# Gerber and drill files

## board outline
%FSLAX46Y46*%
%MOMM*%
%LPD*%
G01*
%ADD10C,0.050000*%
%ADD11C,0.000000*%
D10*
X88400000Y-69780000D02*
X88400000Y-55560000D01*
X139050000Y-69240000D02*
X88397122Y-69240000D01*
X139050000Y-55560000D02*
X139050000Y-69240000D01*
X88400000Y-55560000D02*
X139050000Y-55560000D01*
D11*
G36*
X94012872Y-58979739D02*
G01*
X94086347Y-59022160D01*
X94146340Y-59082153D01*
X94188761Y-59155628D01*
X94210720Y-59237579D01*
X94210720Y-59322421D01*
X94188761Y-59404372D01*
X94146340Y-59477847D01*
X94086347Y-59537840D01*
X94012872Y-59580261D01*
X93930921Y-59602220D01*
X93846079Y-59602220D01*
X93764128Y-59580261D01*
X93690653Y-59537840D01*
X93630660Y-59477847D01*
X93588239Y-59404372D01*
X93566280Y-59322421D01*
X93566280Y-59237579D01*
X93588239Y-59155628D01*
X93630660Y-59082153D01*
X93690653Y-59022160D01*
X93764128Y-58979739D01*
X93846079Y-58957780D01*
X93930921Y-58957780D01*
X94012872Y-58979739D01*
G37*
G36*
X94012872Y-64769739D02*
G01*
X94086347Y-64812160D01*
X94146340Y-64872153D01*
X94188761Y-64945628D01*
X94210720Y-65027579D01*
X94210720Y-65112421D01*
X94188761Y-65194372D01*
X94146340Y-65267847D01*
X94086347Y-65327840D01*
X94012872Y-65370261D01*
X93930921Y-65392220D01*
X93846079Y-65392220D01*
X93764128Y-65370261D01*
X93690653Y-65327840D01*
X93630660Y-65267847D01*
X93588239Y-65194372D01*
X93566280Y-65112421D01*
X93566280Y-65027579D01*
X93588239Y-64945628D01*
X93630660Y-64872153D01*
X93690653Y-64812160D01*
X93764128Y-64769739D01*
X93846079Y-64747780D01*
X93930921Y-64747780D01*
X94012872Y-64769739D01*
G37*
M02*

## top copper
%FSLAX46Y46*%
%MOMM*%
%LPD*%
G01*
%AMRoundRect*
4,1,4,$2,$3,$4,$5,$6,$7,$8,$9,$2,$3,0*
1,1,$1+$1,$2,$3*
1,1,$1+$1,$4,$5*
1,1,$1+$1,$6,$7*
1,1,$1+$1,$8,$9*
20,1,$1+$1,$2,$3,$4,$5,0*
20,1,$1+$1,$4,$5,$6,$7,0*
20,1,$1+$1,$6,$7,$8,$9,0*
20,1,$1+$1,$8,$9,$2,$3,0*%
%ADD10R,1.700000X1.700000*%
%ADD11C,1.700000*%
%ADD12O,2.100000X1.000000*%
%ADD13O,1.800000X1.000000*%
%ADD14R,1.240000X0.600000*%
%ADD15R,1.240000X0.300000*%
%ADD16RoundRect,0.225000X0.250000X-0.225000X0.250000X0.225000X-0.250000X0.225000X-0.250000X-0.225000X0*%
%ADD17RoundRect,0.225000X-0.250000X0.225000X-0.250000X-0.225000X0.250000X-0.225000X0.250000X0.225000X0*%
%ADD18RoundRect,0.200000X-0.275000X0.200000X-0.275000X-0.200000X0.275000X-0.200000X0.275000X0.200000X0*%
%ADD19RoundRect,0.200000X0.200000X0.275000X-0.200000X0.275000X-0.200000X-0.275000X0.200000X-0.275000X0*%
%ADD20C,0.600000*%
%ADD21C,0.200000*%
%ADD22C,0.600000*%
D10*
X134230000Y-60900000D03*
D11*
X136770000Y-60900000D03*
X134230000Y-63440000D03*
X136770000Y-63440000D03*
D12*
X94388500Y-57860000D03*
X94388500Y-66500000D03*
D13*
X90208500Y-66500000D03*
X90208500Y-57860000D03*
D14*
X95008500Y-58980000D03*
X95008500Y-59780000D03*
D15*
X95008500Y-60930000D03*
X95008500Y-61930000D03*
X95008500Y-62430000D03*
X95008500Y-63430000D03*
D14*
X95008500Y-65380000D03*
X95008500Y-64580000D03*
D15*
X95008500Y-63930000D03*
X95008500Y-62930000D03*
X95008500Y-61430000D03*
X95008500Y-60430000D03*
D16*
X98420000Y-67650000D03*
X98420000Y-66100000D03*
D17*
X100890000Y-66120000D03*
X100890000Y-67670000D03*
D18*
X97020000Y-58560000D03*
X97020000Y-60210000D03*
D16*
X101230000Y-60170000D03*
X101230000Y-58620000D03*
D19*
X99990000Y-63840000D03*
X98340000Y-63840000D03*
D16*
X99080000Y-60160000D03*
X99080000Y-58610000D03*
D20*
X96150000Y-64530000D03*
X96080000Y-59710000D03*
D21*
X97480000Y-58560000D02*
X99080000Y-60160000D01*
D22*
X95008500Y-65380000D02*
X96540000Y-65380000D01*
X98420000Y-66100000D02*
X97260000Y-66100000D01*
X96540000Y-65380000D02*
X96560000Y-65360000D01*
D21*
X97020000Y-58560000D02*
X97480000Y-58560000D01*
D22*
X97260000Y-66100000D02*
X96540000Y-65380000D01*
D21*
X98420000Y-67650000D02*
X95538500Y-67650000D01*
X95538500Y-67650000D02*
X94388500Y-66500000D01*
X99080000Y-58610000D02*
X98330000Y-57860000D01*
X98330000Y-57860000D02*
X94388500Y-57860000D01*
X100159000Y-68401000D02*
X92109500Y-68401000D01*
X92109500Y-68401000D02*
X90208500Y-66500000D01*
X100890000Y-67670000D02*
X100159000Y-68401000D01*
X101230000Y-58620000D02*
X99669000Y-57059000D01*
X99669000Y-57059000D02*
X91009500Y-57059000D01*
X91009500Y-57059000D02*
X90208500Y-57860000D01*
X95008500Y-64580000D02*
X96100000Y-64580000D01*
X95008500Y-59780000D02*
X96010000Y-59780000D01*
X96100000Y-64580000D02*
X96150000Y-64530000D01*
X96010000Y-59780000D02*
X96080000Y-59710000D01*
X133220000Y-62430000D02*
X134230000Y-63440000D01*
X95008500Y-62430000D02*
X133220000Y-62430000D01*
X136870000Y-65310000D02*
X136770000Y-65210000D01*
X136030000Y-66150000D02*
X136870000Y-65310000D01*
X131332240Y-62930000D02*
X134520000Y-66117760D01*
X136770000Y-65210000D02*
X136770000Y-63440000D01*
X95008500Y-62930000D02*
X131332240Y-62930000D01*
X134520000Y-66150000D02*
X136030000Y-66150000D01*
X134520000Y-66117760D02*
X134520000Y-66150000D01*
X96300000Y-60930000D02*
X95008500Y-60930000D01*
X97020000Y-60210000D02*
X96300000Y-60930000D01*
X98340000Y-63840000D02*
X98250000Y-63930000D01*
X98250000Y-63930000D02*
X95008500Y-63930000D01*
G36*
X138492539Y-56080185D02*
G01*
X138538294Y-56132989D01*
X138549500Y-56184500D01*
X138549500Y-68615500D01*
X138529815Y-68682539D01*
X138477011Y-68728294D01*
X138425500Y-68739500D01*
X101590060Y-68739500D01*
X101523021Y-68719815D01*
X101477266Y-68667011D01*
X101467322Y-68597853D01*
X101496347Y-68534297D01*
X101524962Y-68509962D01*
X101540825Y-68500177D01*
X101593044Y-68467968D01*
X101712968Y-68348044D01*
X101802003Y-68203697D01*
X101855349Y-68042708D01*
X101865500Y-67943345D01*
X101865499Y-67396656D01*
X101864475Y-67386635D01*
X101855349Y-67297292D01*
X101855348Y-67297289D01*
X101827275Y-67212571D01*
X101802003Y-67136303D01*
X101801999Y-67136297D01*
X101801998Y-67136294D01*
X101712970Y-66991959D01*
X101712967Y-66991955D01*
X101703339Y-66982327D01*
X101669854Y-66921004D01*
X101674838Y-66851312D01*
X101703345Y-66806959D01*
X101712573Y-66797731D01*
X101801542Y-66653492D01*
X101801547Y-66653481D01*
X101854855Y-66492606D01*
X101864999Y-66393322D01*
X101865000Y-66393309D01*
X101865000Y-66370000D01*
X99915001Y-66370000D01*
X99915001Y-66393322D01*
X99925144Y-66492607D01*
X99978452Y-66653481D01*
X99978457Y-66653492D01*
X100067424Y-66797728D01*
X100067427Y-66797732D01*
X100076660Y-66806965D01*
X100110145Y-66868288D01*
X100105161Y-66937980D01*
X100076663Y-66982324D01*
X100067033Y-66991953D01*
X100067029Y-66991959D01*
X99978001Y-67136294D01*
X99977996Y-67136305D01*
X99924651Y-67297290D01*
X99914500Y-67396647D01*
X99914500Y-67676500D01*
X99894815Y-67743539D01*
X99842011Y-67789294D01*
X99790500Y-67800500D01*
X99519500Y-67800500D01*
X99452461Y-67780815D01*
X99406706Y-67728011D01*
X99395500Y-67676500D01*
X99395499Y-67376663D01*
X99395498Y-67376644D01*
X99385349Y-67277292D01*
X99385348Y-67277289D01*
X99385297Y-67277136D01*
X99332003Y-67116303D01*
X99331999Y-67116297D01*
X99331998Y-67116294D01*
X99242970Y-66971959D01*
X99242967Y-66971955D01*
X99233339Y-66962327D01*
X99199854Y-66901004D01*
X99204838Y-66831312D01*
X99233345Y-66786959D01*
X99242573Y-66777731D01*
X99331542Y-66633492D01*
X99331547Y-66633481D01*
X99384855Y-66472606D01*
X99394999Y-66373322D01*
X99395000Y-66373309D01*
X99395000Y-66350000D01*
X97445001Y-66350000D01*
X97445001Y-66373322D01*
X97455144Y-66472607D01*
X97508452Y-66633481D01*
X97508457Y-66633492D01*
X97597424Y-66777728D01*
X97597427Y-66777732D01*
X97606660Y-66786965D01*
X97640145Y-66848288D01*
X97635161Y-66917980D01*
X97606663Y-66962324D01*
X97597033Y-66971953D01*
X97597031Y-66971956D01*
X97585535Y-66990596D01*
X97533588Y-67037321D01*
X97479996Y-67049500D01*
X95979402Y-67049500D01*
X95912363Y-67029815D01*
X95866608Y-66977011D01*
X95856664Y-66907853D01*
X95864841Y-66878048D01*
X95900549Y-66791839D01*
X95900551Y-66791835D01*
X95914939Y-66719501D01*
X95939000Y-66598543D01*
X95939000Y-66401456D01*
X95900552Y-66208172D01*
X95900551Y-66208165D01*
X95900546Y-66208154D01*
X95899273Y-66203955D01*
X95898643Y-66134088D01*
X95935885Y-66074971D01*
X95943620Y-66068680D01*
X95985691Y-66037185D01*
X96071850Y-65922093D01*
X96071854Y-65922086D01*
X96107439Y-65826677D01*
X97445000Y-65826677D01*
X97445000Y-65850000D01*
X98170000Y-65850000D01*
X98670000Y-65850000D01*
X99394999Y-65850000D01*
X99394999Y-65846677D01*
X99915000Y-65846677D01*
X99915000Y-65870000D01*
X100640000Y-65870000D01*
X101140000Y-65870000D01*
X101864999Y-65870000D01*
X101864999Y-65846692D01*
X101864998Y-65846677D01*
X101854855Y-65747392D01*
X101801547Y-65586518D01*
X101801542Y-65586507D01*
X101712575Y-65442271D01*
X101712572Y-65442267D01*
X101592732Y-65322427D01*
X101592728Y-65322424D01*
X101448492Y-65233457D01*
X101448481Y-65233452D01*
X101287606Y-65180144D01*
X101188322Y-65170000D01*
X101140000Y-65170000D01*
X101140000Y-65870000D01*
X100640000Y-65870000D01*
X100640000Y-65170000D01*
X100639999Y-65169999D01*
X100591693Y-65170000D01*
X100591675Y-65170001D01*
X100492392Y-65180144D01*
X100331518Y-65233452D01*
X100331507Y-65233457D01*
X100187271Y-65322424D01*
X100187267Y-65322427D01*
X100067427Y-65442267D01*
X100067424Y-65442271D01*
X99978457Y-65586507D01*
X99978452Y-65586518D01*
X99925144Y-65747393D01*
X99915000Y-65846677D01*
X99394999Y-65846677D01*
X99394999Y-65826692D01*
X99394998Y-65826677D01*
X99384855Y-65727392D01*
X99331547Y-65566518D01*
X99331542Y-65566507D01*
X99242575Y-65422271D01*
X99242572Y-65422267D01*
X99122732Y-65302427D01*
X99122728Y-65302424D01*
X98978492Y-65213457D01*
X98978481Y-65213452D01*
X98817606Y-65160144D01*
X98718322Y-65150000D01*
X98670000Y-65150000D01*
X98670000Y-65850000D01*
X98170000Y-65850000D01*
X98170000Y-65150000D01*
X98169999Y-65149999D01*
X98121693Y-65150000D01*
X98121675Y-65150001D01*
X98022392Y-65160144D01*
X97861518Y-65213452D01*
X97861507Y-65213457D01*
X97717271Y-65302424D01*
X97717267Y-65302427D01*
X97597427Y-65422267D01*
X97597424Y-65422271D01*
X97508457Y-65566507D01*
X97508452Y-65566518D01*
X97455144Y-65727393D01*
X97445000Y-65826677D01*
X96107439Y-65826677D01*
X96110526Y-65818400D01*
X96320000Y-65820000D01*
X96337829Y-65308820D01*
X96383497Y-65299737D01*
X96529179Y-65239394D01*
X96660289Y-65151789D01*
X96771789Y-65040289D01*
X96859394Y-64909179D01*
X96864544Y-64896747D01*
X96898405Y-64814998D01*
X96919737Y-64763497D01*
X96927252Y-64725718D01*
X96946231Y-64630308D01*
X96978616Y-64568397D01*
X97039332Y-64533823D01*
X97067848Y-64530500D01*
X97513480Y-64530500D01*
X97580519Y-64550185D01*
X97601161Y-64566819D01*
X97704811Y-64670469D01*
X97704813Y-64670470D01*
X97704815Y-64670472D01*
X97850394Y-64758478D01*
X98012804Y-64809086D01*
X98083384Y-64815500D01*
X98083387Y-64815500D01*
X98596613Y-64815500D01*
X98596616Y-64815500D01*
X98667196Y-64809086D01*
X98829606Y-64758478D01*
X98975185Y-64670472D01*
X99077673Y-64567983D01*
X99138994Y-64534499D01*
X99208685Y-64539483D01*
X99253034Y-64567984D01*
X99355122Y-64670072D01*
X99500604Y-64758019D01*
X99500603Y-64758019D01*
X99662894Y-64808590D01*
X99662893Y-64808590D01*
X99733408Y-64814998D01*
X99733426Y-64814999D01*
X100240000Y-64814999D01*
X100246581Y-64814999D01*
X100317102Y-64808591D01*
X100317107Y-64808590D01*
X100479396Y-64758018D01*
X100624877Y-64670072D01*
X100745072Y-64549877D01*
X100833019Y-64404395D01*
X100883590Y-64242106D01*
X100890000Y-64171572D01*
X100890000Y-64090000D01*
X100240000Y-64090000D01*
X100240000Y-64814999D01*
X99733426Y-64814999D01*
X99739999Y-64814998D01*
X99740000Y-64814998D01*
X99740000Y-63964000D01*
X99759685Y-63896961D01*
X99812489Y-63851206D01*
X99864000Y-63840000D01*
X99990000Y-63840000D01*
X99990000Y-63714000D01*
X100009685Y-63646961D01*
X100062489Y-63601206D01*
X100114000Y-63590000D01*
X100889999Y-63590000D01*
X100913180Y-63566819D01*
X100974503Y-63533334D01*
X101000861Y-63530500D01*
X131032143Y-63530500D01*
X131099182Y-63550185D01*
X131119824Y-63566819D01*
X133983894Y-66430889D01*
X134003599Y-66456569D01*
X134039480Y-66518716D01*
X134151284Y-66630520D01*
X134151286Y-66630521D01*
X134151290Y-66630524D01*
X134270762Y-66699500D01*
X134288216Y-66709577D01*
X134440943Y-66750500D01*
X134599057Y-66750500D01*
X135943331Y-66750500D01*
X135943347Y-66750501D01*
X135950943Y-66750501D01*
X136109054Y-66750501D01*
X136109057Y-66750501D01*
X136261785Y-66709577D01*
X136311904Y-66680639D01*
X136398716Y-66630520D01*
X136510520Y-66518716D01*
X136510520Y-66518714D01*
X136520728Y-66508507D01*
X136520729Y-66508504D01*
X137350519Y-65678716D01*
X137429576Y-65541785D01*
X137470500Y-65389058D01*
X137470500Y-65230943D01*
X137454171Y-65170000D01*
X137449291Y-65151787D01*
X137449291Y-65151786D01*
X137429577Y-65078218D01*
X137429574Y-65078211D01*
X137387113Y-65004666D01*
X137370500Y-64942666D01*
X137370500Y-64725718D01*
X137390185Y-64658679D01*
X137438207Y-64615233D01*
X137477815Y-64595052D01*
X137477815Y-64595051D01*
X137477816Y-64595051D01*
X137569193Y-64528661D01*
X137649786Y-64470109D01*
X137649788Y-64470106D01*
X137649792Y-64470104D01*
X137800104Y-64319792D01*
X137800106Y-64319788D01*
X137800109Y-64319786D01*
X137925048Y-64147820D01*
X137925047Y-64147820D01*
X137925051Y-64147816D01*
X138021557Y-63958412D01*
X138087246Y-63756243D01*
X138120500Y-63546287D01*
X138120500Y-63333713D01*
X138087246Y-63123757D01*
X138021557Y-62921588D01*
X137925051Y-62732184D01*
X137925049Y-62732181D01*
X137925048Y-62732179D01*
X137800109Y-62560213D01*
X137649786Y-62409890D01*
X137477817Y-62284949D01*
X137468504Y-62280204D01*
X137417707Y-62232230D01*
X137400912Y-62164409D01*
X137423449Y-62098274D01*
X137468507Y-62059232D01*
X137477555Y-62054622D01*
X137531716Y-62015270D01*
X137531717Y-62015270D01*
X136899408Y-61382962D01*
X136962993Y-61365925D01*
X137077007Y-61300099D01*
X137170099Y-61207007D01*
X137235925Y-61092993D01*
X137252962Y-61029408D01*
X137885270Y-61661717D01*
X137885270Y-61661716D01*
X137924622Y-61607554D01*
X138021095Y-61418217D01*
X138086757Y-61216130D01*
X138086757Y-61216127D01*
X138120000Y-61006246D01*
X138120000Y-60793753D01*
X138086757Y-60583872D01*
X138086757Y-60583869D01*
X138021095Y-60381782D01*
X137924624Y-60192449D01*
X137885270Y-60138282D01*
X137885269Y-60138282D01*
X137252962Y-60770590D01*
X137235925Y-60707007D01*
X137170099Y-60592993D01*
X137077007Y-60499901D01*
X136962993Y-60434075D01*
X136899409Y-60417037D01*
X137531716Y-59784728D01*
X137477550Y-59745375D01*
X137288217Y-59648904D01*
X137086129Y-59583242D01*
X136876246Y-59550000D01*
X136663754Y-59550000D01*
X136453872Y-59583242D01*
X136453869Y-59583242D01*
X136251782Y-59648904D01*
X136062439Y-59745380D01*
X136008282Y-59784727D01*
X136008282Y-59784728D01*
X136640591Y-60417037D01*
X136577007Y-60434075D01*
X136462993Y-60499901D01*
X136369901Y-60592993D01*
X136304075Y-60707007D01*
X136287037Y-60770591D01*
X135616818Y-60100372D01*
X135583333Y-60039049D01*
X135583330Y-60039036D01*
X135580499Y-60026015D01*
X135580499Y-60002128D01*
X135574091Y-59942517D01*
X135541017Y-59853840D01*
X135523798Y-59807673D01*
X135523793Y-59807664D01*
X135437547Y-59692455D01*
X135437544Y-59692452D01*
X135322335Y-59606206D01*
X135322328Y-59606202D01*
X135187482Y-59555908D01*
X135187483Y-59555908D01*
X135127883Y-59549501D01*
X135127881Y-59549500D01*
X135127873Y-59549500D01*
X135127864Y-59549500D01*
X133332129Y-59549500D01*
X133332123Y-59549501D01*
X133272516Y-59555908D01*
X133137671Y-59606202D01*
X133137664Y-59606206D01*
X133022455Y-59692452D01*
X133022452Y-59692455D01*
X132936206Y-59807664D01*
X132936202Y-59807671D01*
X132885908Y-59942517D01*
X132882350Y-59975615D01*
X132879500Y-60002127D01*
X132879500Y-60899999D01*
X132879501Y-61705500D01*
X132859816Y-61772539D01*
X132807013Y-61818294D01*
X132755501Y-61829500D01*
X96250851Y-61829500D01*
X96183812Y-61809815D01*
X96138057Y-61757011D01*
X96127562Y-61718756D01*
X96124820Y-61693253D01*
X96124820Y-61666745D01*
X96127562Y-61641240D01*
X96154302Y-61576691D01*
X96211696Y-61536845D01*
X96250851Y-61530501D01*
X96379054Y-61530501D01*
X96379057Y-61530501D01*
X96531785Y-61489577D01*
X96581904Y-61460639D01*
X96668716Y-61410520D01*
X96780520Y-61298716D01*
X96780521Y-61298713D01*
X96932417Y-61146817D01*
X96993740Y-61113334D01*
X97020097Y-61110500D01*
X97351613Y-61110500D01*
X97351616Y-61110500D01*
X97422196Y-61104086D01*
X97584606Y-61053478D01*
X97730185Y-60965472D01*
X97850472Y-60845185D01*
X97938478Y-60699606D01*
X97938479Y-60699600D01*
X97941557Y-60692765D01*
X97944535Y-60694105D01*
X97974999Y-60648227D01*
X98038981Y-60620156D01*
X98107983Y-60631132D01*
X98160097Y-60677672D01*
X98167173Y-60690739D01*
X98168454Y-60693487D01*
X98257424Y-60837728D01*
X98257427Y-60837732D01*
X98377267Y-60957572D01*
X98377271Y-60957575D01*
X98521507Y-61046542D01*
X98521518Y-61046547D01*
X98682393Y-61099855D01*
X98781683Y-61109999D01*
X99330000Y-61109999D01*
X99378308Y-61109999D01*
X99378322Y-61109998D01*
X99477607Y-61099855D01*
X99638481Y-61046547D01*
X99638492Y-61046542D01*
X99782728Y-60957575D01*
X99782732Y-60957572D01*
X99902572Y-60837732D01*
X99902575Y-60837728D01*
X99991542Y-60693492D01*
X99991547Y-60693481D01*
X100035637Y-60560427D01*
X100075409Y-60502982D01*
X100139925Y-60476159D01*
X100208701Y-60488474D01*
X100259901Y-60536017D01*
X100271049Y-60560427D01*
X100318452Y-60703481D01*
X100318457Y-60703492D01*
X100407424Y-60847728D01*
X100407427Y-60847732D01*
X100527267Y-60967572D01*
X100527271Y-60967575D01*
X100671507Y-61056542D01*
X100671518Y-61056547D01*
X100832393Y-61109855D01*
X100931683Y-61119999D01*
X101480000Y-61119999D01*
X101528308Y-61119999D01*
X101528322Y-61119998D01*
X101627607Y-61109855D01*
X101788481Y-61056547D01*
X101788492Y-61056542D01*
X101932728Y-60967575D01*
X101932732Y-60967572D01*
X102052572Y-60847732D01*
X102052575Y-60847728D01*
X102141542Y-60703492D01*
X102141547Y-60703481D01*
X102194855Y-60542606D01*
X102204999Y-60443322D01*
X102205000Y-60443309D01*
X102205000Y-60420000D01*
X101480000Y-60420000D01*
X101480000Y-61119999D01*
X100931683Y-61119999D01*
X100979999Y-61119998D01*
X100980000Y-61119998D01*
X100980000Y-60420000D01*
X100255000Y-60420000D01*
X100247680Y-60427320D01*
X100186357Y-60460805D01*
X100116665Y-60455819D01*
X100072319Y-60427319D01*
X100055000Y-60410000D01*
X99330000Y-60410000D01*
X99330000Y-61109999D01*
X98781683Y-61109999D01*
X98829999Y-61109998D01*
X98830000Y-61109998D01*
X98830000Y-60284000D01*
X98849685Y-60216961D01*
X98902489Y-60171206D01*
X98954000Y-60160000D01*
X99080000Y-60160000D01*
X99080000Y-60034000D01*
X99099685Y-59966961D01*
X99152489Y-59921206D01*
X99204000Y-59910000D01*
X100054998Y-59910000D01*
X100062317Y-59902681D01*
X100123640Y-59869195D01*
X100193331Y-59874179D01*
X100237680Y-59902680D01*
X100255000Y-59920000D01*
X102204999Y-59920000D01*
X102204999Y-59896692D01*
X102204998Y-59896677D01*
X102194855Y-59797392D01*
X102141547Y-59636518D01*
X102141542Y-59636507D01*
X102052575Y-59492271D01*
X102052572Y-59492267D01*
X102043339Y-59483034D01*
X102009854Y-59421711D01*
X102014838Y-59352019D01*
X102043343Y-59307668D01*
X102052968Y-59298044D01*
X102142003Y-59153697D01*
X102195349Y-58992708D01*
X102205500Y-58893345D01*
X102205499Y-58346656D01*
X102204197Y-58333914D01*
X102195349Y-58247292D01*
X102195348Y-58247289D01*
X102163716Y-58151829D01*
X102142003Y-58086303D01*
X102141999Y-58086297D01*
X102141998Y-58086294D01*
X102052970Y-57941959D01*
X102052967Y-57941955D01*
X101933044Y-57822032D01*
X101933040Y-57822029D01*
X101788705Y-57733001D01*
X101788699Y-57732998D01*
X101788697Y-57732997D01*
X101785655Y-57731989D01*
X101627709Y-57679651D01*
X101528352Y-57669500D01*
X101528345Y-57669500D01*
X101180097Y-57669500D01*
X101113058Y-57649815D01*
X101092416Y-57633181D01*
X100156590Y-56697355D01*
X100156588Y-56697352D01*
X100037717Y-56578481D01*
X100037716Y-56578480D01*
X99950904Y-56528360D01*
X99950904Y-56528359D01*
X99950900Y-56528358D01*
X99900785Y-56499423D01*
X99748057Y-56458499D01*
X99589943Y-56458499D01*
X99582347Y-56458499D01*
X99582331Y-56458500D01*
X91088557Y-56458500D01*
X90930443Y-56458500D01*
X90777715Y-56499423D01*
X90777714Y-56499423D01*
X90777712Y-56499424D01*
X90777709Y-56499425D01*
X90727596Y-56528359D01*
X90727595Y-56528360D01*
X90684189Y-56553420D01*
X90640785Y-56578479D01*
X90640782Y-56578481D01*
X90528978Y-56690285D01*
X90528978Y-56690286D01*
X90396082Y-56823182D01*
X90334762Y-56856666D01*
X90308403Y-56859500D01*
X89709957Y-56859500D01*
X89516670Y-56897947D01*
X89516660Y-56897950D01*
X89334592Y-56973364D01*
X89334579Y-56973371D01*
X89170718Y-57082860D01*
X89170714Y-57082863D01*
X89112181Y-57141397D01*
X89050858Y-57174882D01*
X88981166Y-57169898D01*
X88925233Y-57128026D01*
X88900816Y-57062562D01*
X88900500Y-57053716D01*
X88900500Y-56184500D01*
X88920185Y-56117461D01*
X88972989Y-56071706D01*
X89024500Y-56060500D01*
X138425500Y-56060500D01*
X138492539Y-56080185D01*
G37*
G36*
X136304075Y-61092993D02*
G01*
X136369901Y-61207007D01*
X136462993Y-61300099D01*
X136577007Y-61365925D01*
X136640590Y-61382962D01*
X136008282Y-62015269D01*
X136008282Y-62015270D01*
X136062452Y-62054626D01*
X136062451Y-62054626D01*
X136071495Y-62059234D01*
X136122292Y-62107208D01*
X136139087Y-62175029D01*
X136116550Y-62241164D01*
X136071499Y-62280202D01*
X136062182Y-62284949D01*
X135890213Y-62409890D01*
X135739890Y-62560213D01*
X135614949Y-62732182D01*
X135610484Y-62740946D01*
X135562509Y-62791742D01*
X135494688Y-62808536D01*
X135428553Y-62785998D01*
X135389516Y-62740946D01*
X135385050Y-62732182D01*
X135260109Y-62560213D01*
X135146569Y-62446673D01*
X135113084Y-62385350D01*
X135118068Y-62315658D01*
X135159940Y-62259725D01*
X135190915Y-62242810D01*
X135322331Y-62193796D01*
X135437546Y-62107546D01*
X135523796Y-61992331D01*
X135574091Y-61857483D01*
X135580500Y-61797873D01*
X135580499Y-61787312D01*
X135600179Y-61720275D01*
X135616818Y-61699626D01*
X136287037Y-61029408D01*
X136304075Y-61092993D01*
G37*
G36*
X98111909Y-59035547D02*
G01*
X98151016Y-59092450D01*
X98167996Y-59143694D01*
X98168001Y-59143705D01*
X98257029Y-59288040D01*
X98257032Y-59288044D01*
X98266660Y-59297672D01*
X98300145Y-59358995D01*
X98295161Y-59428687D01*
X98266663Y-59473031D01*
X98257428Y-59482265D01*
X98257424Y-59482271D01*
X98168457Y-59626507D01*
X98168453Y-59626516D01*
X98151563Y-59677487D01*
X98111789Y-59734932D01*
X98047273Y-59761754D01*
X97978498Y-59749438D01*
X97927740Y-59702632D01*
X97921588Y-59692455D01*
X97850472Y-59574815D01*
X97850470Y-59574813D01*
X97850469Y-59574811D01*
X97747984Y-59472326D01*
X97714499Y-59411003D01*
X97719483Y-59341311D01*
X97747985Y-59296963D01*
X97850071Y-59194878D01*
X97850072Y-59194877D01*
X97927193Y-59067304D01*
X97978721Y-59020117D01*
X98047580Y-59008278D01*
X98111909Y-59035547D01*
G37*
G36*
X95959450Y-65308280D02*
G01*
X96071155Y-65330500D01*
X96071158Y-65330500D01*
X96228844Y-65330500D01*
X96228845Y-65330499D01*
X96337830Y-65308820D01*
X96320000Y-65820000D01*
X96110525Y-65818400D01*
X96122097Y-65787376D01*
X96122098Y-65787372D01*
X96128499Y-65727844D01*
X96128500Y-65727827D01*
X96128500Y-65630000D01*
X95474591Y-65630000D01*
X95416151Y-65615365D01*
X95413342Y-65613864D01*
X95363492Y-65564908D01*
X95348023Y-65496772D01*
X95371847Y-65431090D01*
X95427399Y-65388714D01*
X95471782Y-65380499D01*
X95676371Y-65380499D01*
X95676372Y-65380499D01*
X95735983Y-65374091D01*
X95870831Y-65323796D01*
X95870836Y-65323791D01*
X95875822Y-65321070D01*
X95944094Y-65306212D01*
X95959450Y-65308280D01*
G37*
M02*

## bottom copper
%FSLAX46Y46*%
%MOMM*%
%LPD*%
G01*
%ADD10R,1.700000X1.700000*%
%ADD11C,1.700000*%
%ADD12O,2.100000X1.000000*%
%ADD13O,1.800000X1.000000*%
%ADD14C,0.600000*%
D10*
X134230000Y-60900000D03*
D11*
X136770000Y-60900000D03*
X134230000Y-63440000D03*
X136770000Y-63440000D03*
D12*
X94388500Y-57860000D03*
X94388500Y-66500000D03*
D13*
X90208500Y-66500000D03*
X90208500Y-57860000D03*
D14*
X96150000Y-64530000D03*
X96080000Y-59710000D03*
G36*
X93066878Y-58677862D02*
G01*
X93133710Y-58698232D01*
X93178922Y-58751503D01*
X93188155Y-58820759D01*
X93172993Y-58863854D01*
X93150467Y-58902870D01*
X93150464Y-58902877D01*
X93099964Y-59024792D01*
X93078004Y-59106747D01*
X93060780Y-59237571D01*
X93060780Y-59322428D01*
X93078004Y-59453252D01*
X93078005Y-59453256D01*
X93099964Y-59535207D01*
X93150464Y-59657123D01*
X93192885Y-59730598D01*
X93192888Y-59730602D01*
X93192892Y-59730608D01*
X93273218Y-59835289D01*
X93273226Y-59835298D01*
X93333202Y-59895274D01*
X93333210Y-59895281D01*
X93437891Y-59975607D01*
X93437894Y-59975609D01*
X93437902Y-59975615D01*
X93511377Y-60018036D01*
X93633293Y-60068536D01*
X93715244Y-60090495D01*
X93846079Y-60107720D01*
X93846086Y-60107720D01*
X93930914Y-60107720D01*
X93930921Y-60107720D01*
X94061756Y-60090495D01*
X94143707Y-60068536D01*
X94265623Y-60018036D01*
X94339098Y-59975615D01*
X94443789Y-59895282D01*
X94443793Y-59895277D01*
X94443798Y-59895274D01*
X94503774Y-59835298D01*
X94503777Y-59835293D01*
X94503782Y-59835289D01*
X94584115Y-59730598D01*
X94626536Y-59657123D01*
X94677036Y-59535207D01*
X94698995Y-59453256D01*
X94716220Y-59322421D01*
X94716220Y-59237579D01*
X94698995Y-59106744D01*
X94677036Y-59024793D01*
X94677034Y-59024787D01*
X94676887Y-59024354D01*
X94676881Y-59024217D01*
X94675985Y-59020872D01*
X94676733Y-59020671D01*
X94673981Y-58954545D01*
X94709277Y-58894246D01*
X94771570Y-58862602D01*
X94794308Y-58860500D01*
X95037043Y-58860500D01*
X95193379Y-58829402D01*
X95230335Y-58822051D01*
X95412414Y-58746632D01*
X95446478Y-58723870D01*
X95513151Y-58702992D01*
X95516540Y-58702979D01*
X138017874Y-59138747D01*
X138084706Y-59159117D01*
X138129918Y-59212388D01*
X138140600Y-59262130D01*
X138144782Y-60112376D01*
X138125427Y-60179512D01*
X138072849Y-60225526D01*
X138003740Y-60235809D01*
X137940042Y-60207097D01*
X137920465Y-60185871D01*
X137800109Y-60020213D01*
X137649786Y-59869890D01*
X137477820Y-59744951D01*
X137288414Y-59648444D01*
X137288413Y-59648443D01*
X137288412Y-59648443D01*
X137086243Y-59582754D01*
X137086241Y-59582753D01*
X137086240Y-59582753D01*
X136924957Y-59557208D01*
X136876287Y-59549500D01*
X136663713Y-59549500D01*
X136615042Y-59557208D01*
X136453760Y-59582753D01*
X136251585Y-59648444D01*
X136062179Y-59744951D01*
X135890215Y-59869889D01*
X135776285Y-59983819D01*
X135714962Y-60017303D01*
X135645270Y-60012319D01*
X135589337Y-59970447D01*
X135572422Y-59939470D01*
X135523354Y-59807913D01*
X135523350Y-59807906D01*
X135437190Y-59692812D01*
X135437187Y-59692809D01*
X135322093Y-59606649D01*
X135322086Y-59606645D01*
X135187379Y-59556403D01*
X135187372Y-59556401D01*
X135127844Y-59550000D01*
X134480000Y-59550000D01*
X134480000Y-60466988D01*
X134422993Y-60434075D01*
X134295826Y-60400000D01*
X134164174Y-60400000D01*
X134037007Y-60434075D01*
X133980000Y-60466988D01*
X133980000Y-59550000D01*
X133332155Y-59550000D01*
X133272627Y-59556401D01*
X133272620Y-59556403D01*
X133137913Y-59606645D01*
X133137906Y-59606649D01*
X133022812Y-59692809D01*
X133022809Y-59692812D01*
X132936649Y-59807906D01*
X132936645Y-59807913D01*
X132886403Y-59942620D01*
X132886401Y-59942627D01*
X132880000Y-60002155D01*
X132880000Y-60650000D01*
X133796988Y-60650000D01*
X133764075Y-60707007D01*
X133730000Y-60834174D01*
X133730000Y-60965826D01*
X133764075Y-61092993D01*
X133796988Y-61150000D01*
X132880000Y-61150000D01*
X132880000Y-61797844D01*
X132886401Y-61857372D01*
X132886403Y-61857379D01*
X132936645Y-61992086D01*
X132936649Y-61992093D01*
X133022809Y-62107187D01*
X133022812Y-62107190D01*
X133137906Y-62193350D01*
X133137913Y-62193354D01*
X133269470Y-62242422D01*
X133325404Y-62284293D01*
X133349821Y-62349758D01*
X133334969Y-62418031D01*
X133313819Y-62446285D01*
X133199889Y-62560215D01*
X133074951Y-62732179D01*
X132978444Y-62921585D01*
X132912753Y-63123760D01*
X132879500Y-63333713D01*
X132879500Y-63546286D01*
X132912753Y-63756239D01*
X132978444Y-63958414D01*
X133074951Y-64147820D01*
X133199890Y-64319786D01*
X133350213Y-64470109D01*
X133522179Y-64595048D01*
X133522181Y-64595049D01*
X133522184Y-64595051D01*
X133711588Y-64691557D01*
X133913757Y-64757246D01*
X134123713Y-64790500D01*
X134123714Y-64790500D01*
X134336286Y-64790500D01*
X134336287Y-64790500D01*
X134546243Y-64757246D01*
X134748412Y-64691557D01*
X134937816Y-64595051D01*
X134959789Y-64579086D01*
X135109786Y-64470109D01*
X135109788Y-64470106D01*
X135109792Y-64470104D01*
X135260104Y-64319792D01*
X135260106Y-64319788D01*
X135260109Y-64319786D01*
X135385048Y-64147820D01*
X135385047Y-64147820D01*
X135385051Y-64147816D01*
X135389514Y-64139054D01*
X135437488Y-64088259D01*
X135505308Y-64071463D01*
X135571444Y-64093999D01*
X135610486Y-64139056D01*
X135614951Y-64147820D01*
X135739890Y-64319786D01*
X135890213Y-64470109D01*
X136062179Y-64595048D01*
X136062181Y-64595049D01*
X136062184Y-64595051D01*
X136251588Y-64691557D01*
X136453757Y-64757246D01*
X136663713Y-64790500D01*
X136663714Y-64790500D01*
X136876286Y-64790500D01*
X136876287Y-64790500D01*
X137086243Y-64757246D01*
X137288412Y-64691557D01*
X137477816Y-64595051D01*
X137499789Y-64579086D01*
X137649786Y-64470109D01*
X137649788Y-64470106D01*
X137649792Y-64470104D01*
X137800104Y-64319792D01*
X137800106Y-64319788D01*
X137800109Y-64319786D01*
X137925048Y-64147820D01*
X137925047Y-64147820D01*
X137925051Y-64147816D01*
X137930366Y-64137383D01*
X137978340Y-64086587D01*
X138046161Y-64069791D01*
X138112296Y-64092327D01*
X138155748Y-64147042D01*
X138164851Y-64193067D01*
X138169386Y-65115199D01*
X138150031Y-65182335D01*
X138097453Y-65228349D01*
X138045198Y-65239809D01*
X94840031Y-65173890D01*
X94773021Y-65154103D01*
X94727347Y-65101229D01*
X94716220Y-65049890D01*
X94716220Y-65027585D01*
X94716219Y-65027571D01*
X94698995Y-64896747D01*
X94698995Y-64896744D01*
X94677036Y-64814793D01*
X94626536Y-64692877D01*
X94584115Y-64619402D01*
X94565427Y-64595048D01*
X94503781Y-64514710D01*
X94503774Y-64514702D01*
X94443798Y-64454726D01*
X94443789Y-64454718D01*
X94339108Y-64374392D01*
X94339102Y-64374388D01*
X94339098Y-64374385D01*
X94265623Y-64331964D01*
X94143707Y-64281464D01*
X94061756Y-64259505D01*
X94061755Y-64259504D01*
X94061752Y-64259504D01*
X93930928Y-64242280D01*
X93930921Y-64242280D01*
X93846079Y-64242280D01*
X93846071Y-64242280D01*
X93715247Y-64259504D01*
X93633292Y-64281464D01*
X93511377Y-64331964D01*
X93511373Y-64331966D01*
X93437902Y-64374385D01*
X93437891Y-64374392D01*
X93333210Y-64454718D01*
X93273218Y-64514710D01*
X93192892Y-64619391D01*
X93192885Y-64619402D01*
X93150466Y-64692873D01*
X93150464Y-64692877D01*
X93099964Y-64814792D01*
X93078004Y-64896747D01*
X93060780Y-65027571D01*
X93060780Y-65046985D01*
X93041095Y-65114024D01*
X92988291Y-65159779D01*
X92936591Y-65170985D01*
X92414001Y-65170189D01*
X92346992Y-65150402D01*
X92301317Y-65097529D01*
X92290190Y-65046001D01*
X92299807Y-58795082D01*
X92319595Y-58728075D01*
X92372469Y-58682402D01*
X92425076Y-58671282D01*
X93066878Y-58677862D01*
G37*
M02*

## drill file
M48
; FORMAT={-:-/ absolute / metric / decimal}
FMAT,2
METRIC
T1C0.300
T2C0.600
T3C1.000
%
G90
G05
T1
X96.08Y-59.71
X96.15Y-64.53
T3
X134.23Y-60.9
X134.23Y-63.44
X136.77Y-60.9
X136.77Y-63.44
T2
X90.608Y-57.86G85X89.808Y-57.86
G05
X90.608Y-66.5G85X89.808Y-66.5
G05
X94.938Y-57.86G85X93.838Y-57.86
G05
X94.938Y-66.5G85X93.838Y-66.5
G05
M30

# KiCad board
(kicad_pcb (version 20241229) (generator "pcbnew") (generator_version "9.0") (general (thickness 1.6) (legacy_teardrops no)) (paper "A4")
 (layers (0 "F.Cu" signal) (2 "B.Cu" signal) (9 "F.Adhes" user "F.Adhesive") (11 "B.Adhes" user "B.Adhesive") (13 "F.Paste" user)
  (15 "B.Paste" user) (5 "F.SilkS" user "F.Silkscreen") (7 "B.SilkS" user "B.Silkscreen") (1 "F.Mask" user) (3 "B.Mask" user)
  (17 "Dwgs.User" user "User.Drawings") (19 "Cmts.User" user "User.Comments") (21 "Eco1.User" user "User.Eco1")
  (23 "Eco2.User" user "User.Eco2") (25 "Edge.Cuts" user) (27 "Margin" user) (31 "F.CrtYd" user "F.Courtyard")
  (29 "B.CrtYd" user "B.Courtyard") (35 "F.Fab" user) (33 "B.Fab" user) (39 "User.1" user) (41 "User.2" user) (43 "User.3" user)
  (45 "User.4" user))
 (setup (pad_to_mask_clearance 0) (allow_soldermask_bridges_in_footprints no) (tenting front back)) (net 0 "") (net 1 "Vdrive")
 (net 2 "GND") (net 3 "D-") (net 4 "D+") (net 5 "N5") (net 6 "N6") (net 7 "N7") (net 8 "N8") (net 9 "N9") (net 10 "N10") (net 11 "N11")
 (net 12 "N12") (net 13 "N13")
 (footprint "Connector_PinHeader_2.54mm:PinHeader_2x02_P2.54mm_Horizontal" (layer "F.Cu") (at 134.23 60.9)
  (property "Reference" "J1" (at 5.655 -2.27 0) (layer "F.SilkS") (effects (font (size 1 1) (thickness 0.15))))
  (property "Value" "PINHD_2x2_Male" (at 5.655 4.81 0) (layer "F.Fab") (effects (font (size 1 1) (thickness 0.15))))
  (pad "1" thru_hole rect (at 0 0) (size 1.7 1.7) (drill 1) (layers "*.Cu" "*.Mask") (remove_unused_layers no) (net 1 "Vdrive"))
  (pad "2" thru_hole circle (at 2.54 0) (size 1.7 1.7) (drill 1) (layers "*.Cu" "*.Mask") (remove_unused_layers no) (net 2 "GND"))
  (pad "3" thru_hole circle (at 0 2.54) (size 1.7 1.7) (drill 1) (layers "*.Cu" "*.Mask") (remove_unused_layers no) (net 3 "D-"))
  (pad "4" thru_hole circle (at 2.54 2.54) (size 1.7 1.7) (drill 1) (layers "*.Cu" "*.Mask") (remove_unused_layers no) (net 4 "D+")))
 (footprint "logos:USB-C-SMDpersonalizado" (layer "F.Cu") (at 92.6085 62.18 -90)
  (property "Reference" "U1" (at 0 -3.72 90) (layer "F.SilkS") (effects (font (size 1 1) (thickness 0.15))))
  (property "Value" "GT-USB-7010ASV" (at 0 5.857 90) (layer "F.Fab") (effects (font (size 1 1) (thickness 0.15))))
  (fp_poly
   (pts (xy -2.57778 -1.322421) (xy -2.599739 -1.404372) (xy -2.64216 -1.477847) (xy -2.702153 -1.53784) (xy -2.775628 -1.580261)
    (xy -2.857579 -1.60222) (xy -2.942421 -1.60222) (xy -3.024372 -1.580261) (xy -3.097847 -1.53784) (xy -3.15784 -1.477847)
    (xy -3.200261 -1.404372) (xy -3.22222 -1.322421) (xy -3.22222 -1.237579) (xy -3.200261 -1.155628) (xy -3.15784 -1.082153)
    (xy -3.097847 -1.02216) (xy -3.024372 -0.979739) (xy -2.942421 -0.95778) (xy -2.857579 -0.95778) (xy -2.775628 -0.979739)
    (xy -2.702153 -1.02216) (xy -2.64216 -1.082153) (xy -2.599739 -1.155628) (xy -2.57778 -1.237579))
   (stroke (width 0) (type default)) (fill yes) (layer "Edge.Cuts"))
  (fp_poly
   (pts (xy 3.21222 -1.322421) (xy 3.190261 -1.404372) (xy 3.14784 -1.477847) (xy 3.087847 -1.53784) (xy 3.014372 -1.580261)
    (xy 2.932421 -1.60222) (xy 2.847579 -1.60222) (xy 2.765628 -1.580261) (xy 2.692153 -1.53784) (xy 2.63216 -1.477847)
    (xy 2.589739 -1.404372) (xy 2.56778 -1.322421) (xy 2.56778 -1.237579) (xy 2.589739 -1.155628) (xy 2.63216 -1.082153)
    (xy 2.692153 -1.02216) (xy 2.765628 -0.979739) (xy 2.847579 -0.95778) (xy 2.932421 -0.95778) (xy 3.014372 -0.979739)
    (xy 3.087847 -1.02216) (xy 3.14784 -1.082153) (xy 3.190261 -1.155628) (xy 3.21222 -1.237579))
   (stroke (width 0) (type default)) (fill yes) (layer "Edge.Cuts"))
  (pad "1" thru_hole oval (at -4.32 -1.78 270) (size 1 2.1) (drill oval 0.6 1.7) (layers "*.Cu" "*.Mask") (remove_unused_layers no)
   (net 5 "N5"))
  (pad "2" thru_hole oval (at 4.32 -1.78 270) (size 1 2.1) (drill oval 0.6 1.7) (layers "*.Cu" "*.Mask") (remove_unused_layers no)
   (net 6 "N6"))
  (pad "3" thru_hole oval (at 4.32 2.4 270) (size 1 1.8) (drill oval 0.6 1.4) (layers "*.Cu" "*.Mask") (remove_unused_layers no)
   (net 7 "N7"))
  (pad "4" thru_hole oval (at -4.32 2.4 270) (size 1 1.8) (drill oval 0.6 1.4) (layers "*.Cu" "*.Mask") (remove_unused_layers no)
   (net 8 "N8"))
  (pad "A1B12" smd rect (at -3.2 -2.4 270) (size 0.6 1.24) (layers "F.Cu" "F.Mask" "F.Paste") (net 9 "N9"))
  (pad "A4B9" smd rect (at -2.4 -2.4 270) (size 0.6 1.24) (layers "F.Cu" "F.Mask" "F.Paste") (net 1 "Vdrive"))
  (pad "A5" smd rect (at -1.25 -2.4 270) (size 0.3 1.24) (layers "F.Cu" "F.Mask" "F.Paste") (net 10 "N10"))
  (pad "A6" smd rect (at -0.25 -2.4 270) (size 0.3 1.24) (layers "F.Cu" "F.Mask" "F.Paste") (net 4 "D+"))
  (pad "A7" smd rect (at 0.25 -2.4 270) (size 0.3 1.24) (layers "F.Cu" "F.Mask" "F.Paste") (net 3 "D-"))
  (pad "A8" smd rect (at 1.25 -2.4 270) (size 0.3 1.24) (layers "F.Cu" "F.Mask" "F.Paste") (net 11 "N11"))
  (pad "B1A12" smd rect (at 3.2 -2.4 270) (size 0.6 1.24) (layers "F.Cu" "F.Mask" "F.Paste") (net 2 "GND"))
  (pad "B4A9" smd rect (at 2.4 -2.4 270) (size 0.6 1.24) (layers "F.Cu" "F.Mask" "F.Paste") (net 1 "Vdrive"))
  (pad "B5" smd rect (at 1.75 -2.4 270) (size 0.3 1.24) (layers "F.Cu" "F.Mask" "F.Paste") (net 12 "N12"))
  (pad "B6" smd rect (at 0.75 -2.4 270) (size 0.3 1.24) (layers "F.Cu" "F.Mask" "F.Paste") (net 4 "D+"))
  (pad "B7" smd rect (at -0.75 -2.4 270) (size 0.3 1.24) (layers "F.Cu" "F.Mask" "F.Paste") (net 3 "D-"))
  (pad "B8" smd rect (at -1.75 -2.4 270) (size 0.3 1.24) (layers "F.Cu" "F.Mask" "F.Paste") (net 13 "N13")))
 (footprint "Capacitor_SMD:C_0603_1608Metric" (layer "F.Cu") (at 98.42 66.875 90)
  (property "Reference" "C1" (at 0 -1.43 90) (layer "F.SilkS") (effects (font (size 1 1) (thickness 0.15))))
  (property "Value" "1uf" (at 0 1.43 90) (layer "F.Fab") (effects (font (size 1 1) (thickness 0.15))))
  (pad "1" smd roundrect (at -0.775 0 90) (size 0.9 0.95) (layers "F.Cu" "F.Mask" "F.Paste") (roundrect_rratio 0.25) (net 6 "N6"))
  (pad "2" smd roundrect (at 0.775 0 90) (size 0.9 0.95) (layers "F.Cu" "F.Mask" "F.Paste") (roundrect_rratio 0.25) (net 2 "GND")))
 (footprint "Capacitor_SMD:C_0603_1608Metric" (layer "F.Cu") (at 100.89 66.895 -90)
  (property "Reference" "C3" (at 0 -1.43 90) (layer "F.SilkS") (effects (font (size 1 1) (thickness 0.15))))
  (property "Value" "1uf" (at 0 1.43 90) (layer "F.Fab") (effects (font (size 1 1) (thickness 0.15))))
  (pad "1" smd roundrect (at -0.775 0 270) (size 0.9 0.95) (layers "F.Cu" "F.Mask" "F.Paste") (roundrect_rratio 0.25) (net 2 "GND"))
  (pad "2" smd roundrect (at 0.775 0 270) (size 0.9 0.95) (layers "F.Cu" "F.Mask" "F.Paste") (roundrect_rratio 0.25) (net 7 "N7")))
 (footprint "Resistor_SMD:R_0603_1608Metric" (layer "F.Cu") (at 97.02 59.385 -90)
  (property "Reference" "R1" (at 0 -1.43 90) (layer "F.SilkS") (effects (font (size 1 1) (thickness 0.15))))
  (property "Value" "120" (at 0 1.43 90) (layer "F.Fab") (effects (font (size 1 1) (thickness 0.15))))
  (pad "1" smd roundrect (at -0.825 0 270) (size 0.8 0.95) (layers "F.Cu" "F.Mask" "F.Paste") (roundrect_rratio 0.25) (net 2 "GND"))
  (pad "2" smd roundrect (at 0.825 0 270) (size 0.8 0.95) (layers "F.Cu" "F.Mask" "F.Paste") (roundrect_rratio 0.25) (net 10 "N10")))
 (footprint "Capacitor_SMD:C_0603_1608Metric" (layer "F.Cu") (at 101.23 59.395 90)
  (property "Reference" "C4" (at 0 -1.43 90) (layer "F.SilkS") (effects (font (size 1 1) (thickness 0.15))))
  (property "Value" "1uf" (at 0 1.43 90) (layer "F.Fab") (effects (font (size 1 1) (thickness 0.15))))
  (pad "1" smd roundrect (at -0.775 0 90) (size 0.9 0.95) (layers "F.Cu" "F.Mask" "F.Paste") (roundrect_rratio 0.25) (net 2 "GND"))
  (pad "2" smd roundrect (at 0.775 0 90) (size 0.9 0.95) (layers "F.Cu" "F.Mask" "F.Paste") (roundrect_rratio 0.25) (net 8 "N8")))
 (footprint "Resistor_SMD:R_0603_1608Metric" (layer "F.Cu") (at 99.165 63.84 180)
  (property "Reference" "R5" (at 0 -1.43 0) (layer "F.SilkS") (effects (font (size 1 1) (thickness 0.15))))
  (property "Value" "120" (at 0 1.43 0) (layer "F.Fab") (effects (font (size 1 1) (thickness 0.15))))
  (pad "1" smd roundrect (at -0.825 0 180) (size 0.8 0.95) (layers "F.Cu" "F.Mask" "F.Paste") (roundrect_rratio 0.25) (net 2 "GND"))
  (pad "2" smd roundrect (at 0.825 0 180) (size 0.8 0.95) (layers "F.Cu" "F.Mask" "F.Paste") (roundrect_rratio 0.25) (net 12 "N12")))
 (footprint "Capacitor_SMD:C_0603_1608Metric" (layer "F.Cu") (at 99.08 59.385 90)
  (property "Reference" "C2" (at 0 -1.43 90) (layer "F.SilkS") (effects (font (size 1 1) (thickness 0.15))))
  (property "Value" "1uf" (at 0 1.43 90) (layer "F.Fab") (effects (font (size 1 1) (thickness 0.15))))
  (pad "1" smd roundrect (at -0.775 0 90) (size 0.9 0.95) (layers "F.Cu" "F.Mask" "F.Paste") (roundrect_rratio 0.25) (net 2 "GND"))
  (pad "2" smd roundrect (at 0.775 0 90) (size 0.9 0.95) (layers "F.Cu" "F.Mask" "F.Paste") (roundrect_rratio 0.25) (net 5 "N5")))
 (gr_line (start 88.4 69.78) (end 88.4 55.56) (stroke (width 0.05) (type default)) (layer "Edge.Cuts"))
 (gr_line (start 139.05 69.24) (end 88.397122 69.24) (stroke (width 0.05) (type solid)) (layer "Edge.Cuts"))
 (gr_line (start 139.05 55.56) (end 139.05 69.24) (stroke (width 0.05) (type default)) (layer "Edge.Cuts"))
 (gr_line (start 88.4 55.56) (end 139.05 55.56) (stroke (width 0.05) (type default)) (layer "Edge.Cuts"))
 (segment (start 97.48 58.56) (end 99.08 60.16) (width 0.2) (layer "F.Cu") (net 2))
 (segment (start 95.0085 65.38) (end 96.54 65.38) (width 0.6) (layer "F.Cu") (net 2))
 (segment (start 98.42 66.1) (end 97.26 66.1) (width 0.6) (layer "F.Cu") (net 2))
 (segment (start 96.54 65.38) (end 96.56 65.36) (width 0.6) (layer "F.Cu") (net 2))
 (segment (start 97.02 58.56) (end 97.48 58.56) (width 0.2) (layer "F.Cu") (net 2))
 (segment (start 97.26 66.1) (end 96.54 65.38) (width 0.6) (layer "F.Cu") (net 2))
 (segment (start 98.42 67.65) (end 95.5385 67.65) (width 0.2) (layer "F.Cu") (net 6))
 (segment (start 95.5385 67.65) (end 94.3885 66.5) (width 0.2) (layer "F.Cu") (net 6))
 (segment (start 99.08 58.61) (end 98.33 57.86) (width 0.2) (layer "F.Cu") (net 5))
 (segment (start 98.33 57.86) (end 94.3885 57.86) (width 0.2) (layer "F.Cu") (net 5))
 (segment (start 100.159 68.401) (end 92.1095 68.401) (width 0.2) (layer "F.Cu") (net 7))
 (segment (start 92.1095 68.401) (end 90.2085 66.5) (width 0.2) (layer "F.Cu") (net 7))
 (segment (start 100.89 67.67) (end 100.159 68.401) (width 0.2) (layer "F.Cu") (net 7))
 (segment (start 101.23 58.62) (end 99.669 57.059) (width 0.2) (layer "F.Cu") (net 8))
 (segment (start 99.669 57.059) (end 91.0095 57.059) (width 0.2) (layer "F.Cu") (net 8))
 (segment (start 91.0095 57.059) (end 90.2085 57.86) (width 0.2) (layer "F.Cu") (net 8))
 (segment (start 95.0085 64.58) (end 96.1 64.58) (width 0.2) (layer "F.Cu") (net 1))
 (segment (start 95.0085 59.78) (end 96.01 59.78) (width 0.2) (layer "F.Cu") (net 1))
 (segment (start 96.1 64.58) (end 96.15 64.53) (width 0.2) (layer "F.Cu") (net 1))
 (segment (start 96.01 59.78) (end 96.08 59.71) (width 0.2) (layer "F.Cu") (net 1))
 (via (at 96.15 64.53) (size 0.6) (drill 0.3) (layers "F.Cu" "B.Cu") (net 1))
 (via (at 96.08 59.71) (size 0.6) (drill 0.3) (layers "F.Cu" "B.Cu") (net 1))
 (segment (start 133.22 62.43) (end 134.23 63.44) (width 0.2) (layer "F.Cu") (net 3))
 (segment (start 95.0085 62.43) (end 133.22 62.43) (width 0.2) (layer "F.Cu") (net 3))
 (segment (start 136.87 65.31) (end 136.77 65.21) (width 0.2) (layer "F.Cu") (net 4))
 (segment (start 136.03 66.15) (end 136.87 65.31) (width 0.2) (layer "F.Cu") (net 4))
 (segment (start 131.33224 62.93) (end 134.52 66.11776) (width 0.2) (layer "F.Cu") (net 4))
 (segment (start 136.77 65.21) (end 136.77 63.44) (width 0.2) (layer "F.Cu") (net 4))
 (segment (start 95.0085 62.93) (end 131.33224 62.93) (width 0.2) (layer "F.Cu") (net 4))
 (segment (start 134.52 66.15) (end 136.03 66.15) (width 0.2) (layer "F.Cu") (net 4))
 (segment (start 134.52 66.11776) (end 134.52 66.15) (width 0.2) (layer "F.Cu") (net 4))
 (segment (start 96.3 60.93) (end 95.0085 60.93) (width 0.2) (layer "F.Cu") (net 10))
 (segment (start 97.02 60.21) (end 96.3 60.93) (width 0.2) (layer "F.Cu") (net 10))
 (segment (start 98.34 63.84) (end 98.25 63.93) (width 0.2) (layer "F.Cu") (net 12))
 (segment (start 98.25 63.93) (end 95.0085 63.93) (width 0.2) (layer "F.Cu") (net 12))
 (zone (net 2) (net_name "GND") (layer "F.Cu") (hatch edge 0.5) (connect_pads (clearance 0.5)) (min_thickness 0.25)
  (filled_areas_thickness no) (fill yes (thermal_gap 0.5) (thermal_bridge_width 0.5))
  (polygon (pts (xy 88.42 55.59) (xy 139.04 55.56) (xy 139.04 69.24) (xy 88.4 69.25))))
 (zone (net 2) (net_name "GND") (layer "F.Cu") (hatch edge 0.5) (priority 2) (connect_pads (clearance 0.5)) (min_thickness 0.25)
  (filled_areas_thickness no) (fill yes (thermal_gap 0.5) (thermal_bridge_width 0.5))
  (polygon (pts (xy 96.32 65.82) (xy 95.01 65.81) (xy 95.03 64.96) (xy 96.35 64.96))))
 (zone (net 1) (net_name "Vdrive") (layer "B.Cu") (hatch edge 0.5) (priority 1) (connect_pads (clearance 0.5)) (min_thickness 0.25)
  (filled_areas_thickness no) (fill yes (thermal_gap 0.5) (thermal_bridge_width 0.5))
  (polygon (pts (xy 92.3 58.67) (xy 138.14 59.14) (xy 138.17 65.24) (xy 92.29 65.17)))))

